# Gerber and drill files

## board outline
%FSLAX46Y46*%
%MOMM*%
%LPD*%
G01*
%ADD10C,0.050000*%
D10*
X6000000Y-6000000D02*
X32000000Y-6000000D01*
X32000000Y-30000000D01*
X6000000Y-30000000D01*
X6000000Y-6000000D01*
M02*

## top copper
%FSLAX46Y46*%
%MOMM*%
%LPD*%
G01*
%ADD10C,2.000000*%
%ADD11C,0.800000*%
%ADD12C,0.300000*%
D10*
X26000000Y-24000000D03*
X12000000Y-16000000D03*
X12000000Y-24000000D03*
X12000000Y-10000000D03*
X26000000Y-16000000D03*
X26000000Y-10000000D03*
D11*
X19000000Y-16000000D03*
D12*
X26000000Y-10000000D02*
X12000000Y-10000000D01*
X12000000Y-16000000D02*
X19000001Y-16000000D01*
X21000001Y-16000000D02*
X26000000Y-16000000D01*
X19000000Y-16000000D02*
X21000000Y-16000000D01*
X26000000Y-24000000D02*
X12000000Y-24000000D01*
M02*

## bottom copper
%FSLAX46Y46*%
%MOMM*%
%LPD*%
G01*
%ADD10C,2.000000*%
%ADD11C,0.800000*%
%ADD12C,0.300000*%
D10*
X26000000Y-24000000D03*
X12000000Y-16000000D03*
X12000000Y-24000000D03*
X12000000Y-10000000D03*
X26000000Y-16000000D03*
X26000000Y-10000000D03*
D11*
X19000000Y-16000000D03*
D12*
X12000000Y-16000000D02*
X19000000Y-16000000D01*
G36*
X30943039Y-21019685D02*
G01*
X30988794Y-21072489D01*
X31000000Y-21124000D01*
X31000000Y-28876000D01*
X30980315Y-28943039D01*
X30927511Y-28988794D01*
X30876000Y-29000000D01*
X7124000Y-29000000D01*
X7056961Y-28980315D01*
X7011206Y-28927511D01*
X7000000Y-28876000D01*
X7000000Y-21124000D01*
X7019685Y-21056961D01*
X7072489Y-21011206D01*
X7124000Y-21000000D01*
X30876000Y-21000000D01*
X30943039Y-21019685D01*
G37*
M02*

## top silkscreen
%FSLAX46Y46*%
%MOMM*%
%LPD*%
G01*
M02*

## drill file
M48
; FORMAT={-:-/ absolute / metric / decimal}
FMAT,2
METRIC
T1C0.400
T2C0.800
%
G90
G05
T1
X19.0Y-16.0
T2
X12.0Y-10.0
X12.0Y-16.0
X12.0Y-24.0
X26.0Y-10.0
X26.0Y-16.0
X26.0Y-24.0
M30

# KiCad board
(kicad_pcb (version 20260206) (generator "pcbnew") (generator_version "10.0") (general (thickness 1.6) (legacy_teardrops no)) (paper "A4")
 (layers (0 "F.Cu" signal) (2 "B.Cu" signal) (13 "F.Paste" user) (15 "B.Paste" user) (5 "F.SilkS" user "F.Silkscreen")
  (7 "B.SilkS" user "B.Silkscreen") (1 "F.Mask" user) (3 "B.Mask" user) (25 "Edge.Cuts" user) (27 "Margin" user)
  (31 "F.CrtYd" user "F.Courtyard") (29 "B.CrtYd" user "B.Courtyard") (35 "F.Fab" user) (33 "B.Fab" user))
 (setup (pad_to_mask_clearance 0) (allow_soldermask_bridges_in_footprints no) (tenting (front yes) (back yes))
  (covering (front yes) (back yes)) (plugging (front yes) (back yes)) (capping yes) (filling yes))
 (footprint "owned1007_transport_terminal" (layer "F.Cu") (at 26 24)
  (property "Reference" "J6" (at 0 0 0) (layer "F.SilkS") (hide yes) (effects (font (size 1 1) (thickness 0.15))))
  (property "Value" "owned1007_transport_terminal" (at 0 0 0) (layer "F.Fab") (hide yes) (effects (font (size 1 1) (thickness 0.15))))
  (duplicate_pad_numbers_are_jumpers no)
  (pad "1" thru_hole circle (at 0 0) (size 2 2) (drill 0.8) (layers "*.Cu" "*.Mask") (remove_unused_layers no) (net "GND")))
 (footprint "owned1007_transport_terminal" (layer "F.Cu") (at 12 16)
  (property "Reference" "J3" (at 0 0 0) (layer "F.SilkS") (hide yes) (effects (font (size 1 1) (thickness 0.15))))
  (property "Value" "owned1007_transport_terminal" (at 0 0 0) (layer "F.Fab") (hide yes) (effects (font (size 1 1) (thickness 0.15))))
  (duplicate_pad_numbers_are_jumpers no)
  (pad "1" thru_hole circle (at 0 0) (size 2 2) (drill 0.8) (layers "*.Cu" "*.Mask") (remove_unused_layers no) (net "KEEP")))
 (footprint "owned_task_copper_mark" (layer "F.Cu") (at 10 28)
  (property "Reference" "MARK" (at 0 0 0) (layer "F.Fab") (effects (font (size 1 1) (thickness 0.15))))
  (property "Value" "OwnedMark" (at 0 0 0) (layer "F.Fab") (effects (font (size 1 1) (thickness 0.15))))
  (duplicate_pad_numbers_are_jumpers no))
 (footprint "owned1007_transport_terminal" (layer "F.Cu") (at 12 24)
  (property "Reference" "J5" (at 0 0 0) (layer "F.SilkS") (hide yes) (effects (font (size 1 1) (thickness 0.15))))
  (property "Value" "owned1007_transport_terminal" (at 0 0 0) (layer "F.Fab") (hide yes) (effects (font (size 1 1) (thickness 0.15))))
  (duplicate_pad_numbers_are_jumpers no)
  (pad "1" thru_hole circle (at 0 0) (size 2 2) (drill 0.8) (layers "*.Cu" "*.Mask") (remove_unused_layers no) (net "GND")))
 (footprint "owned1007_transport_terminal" (layer "F.Cu") (at 12 10)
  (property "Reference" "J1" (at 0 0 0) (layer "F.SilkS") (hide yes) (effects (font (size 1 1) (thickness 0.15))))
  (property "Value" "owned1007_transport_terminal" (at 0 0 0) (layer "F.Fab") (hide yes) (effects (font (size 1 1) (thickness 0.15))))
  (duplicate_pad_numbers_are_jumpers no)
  (pad "1" thru_hole circle (at 0 0) (size 2 2) (drill 0.8) (layers "*.Cu" "*.Mask") (remove_unused_layers no) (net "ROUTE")))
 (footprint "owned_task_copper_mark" (layer "F.Cu") (at 13 28)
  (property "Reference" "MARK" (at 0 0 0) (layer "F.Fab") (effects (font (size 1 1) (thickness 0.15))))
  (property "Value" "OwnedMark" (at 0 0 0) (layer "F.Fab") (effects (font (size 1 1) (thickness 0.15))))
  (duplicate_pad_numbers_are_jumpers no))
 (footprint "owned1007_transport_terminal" (layer "F.Cu") (at 26 16)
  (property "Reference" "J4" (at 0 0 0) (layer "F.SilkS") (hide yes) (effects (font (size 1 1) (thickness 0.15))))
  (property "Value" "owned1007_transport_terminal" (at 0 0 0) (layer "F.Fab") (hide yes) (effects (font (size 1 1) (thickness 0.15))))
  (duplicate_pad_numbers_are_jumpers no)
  (pad "1" thru_hole circle (at 0 0) (size 2 2) (drill 0.8) (layers "*.Cu" "*.Mask") (remove_unused_layers no) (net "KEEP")))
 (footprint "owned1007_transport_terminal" (layer "F.Cu") (at 26 10)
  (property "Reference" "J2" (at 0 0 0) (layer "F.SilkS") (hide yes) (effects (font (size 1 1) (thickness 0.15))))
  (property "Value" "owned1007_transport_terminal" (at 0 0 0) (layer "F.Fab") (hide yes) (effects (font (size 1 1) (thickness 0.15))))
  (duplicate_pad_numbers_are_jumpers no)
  (pad "1" thru_hole circle (at 0 0) (size 2 2) (drill 0.8) (layers "*.Cu" "*.Mask") (remove_unused_layers no) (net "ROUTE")))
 (gr_rect (start 6 6) (end 32 30) (stroke (width 0.05) (type default)) (fill no) (layer "Edge.Cuts"))
 (segment (start 26 10) (end 12 10) (width 0.3) (layer "F.Cu") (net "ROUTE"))
 (segment (start 12 16) (end 19.000001 16) (width 0.3) (layer "F.Cu") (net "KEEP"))
 (segment (start 21.000001 16) (end 26 16) (width 0.3) (layer "F.Cu") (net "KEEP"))
 (segment (start 19 16) (end 21 16) (width 0.3) (layer "F.Cu") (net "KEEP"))
 (via (at 19 16) (size 0.8) (drill 0.4) (layers "F.Cu" "B.Cu") (free yes) (capping no) (covering (front no) (back no))
  (plugging (front no) (back no)) (filling no) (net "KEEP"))
 (segment (start 12 16) (end 19 16) (width 0.3) (locked yes) (layer "B.Cu") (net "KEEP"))
 (segment (start 26 24) (end 12 24) (width 0.3) (layer "F.Cu") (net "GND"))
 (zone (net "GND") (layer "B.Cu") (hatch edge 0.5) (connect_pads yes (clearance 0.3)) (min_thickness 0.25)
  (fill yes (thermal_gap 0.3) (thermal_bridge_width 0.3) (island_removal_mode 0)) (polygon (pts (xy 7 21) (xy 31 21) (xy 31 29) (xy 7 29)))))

